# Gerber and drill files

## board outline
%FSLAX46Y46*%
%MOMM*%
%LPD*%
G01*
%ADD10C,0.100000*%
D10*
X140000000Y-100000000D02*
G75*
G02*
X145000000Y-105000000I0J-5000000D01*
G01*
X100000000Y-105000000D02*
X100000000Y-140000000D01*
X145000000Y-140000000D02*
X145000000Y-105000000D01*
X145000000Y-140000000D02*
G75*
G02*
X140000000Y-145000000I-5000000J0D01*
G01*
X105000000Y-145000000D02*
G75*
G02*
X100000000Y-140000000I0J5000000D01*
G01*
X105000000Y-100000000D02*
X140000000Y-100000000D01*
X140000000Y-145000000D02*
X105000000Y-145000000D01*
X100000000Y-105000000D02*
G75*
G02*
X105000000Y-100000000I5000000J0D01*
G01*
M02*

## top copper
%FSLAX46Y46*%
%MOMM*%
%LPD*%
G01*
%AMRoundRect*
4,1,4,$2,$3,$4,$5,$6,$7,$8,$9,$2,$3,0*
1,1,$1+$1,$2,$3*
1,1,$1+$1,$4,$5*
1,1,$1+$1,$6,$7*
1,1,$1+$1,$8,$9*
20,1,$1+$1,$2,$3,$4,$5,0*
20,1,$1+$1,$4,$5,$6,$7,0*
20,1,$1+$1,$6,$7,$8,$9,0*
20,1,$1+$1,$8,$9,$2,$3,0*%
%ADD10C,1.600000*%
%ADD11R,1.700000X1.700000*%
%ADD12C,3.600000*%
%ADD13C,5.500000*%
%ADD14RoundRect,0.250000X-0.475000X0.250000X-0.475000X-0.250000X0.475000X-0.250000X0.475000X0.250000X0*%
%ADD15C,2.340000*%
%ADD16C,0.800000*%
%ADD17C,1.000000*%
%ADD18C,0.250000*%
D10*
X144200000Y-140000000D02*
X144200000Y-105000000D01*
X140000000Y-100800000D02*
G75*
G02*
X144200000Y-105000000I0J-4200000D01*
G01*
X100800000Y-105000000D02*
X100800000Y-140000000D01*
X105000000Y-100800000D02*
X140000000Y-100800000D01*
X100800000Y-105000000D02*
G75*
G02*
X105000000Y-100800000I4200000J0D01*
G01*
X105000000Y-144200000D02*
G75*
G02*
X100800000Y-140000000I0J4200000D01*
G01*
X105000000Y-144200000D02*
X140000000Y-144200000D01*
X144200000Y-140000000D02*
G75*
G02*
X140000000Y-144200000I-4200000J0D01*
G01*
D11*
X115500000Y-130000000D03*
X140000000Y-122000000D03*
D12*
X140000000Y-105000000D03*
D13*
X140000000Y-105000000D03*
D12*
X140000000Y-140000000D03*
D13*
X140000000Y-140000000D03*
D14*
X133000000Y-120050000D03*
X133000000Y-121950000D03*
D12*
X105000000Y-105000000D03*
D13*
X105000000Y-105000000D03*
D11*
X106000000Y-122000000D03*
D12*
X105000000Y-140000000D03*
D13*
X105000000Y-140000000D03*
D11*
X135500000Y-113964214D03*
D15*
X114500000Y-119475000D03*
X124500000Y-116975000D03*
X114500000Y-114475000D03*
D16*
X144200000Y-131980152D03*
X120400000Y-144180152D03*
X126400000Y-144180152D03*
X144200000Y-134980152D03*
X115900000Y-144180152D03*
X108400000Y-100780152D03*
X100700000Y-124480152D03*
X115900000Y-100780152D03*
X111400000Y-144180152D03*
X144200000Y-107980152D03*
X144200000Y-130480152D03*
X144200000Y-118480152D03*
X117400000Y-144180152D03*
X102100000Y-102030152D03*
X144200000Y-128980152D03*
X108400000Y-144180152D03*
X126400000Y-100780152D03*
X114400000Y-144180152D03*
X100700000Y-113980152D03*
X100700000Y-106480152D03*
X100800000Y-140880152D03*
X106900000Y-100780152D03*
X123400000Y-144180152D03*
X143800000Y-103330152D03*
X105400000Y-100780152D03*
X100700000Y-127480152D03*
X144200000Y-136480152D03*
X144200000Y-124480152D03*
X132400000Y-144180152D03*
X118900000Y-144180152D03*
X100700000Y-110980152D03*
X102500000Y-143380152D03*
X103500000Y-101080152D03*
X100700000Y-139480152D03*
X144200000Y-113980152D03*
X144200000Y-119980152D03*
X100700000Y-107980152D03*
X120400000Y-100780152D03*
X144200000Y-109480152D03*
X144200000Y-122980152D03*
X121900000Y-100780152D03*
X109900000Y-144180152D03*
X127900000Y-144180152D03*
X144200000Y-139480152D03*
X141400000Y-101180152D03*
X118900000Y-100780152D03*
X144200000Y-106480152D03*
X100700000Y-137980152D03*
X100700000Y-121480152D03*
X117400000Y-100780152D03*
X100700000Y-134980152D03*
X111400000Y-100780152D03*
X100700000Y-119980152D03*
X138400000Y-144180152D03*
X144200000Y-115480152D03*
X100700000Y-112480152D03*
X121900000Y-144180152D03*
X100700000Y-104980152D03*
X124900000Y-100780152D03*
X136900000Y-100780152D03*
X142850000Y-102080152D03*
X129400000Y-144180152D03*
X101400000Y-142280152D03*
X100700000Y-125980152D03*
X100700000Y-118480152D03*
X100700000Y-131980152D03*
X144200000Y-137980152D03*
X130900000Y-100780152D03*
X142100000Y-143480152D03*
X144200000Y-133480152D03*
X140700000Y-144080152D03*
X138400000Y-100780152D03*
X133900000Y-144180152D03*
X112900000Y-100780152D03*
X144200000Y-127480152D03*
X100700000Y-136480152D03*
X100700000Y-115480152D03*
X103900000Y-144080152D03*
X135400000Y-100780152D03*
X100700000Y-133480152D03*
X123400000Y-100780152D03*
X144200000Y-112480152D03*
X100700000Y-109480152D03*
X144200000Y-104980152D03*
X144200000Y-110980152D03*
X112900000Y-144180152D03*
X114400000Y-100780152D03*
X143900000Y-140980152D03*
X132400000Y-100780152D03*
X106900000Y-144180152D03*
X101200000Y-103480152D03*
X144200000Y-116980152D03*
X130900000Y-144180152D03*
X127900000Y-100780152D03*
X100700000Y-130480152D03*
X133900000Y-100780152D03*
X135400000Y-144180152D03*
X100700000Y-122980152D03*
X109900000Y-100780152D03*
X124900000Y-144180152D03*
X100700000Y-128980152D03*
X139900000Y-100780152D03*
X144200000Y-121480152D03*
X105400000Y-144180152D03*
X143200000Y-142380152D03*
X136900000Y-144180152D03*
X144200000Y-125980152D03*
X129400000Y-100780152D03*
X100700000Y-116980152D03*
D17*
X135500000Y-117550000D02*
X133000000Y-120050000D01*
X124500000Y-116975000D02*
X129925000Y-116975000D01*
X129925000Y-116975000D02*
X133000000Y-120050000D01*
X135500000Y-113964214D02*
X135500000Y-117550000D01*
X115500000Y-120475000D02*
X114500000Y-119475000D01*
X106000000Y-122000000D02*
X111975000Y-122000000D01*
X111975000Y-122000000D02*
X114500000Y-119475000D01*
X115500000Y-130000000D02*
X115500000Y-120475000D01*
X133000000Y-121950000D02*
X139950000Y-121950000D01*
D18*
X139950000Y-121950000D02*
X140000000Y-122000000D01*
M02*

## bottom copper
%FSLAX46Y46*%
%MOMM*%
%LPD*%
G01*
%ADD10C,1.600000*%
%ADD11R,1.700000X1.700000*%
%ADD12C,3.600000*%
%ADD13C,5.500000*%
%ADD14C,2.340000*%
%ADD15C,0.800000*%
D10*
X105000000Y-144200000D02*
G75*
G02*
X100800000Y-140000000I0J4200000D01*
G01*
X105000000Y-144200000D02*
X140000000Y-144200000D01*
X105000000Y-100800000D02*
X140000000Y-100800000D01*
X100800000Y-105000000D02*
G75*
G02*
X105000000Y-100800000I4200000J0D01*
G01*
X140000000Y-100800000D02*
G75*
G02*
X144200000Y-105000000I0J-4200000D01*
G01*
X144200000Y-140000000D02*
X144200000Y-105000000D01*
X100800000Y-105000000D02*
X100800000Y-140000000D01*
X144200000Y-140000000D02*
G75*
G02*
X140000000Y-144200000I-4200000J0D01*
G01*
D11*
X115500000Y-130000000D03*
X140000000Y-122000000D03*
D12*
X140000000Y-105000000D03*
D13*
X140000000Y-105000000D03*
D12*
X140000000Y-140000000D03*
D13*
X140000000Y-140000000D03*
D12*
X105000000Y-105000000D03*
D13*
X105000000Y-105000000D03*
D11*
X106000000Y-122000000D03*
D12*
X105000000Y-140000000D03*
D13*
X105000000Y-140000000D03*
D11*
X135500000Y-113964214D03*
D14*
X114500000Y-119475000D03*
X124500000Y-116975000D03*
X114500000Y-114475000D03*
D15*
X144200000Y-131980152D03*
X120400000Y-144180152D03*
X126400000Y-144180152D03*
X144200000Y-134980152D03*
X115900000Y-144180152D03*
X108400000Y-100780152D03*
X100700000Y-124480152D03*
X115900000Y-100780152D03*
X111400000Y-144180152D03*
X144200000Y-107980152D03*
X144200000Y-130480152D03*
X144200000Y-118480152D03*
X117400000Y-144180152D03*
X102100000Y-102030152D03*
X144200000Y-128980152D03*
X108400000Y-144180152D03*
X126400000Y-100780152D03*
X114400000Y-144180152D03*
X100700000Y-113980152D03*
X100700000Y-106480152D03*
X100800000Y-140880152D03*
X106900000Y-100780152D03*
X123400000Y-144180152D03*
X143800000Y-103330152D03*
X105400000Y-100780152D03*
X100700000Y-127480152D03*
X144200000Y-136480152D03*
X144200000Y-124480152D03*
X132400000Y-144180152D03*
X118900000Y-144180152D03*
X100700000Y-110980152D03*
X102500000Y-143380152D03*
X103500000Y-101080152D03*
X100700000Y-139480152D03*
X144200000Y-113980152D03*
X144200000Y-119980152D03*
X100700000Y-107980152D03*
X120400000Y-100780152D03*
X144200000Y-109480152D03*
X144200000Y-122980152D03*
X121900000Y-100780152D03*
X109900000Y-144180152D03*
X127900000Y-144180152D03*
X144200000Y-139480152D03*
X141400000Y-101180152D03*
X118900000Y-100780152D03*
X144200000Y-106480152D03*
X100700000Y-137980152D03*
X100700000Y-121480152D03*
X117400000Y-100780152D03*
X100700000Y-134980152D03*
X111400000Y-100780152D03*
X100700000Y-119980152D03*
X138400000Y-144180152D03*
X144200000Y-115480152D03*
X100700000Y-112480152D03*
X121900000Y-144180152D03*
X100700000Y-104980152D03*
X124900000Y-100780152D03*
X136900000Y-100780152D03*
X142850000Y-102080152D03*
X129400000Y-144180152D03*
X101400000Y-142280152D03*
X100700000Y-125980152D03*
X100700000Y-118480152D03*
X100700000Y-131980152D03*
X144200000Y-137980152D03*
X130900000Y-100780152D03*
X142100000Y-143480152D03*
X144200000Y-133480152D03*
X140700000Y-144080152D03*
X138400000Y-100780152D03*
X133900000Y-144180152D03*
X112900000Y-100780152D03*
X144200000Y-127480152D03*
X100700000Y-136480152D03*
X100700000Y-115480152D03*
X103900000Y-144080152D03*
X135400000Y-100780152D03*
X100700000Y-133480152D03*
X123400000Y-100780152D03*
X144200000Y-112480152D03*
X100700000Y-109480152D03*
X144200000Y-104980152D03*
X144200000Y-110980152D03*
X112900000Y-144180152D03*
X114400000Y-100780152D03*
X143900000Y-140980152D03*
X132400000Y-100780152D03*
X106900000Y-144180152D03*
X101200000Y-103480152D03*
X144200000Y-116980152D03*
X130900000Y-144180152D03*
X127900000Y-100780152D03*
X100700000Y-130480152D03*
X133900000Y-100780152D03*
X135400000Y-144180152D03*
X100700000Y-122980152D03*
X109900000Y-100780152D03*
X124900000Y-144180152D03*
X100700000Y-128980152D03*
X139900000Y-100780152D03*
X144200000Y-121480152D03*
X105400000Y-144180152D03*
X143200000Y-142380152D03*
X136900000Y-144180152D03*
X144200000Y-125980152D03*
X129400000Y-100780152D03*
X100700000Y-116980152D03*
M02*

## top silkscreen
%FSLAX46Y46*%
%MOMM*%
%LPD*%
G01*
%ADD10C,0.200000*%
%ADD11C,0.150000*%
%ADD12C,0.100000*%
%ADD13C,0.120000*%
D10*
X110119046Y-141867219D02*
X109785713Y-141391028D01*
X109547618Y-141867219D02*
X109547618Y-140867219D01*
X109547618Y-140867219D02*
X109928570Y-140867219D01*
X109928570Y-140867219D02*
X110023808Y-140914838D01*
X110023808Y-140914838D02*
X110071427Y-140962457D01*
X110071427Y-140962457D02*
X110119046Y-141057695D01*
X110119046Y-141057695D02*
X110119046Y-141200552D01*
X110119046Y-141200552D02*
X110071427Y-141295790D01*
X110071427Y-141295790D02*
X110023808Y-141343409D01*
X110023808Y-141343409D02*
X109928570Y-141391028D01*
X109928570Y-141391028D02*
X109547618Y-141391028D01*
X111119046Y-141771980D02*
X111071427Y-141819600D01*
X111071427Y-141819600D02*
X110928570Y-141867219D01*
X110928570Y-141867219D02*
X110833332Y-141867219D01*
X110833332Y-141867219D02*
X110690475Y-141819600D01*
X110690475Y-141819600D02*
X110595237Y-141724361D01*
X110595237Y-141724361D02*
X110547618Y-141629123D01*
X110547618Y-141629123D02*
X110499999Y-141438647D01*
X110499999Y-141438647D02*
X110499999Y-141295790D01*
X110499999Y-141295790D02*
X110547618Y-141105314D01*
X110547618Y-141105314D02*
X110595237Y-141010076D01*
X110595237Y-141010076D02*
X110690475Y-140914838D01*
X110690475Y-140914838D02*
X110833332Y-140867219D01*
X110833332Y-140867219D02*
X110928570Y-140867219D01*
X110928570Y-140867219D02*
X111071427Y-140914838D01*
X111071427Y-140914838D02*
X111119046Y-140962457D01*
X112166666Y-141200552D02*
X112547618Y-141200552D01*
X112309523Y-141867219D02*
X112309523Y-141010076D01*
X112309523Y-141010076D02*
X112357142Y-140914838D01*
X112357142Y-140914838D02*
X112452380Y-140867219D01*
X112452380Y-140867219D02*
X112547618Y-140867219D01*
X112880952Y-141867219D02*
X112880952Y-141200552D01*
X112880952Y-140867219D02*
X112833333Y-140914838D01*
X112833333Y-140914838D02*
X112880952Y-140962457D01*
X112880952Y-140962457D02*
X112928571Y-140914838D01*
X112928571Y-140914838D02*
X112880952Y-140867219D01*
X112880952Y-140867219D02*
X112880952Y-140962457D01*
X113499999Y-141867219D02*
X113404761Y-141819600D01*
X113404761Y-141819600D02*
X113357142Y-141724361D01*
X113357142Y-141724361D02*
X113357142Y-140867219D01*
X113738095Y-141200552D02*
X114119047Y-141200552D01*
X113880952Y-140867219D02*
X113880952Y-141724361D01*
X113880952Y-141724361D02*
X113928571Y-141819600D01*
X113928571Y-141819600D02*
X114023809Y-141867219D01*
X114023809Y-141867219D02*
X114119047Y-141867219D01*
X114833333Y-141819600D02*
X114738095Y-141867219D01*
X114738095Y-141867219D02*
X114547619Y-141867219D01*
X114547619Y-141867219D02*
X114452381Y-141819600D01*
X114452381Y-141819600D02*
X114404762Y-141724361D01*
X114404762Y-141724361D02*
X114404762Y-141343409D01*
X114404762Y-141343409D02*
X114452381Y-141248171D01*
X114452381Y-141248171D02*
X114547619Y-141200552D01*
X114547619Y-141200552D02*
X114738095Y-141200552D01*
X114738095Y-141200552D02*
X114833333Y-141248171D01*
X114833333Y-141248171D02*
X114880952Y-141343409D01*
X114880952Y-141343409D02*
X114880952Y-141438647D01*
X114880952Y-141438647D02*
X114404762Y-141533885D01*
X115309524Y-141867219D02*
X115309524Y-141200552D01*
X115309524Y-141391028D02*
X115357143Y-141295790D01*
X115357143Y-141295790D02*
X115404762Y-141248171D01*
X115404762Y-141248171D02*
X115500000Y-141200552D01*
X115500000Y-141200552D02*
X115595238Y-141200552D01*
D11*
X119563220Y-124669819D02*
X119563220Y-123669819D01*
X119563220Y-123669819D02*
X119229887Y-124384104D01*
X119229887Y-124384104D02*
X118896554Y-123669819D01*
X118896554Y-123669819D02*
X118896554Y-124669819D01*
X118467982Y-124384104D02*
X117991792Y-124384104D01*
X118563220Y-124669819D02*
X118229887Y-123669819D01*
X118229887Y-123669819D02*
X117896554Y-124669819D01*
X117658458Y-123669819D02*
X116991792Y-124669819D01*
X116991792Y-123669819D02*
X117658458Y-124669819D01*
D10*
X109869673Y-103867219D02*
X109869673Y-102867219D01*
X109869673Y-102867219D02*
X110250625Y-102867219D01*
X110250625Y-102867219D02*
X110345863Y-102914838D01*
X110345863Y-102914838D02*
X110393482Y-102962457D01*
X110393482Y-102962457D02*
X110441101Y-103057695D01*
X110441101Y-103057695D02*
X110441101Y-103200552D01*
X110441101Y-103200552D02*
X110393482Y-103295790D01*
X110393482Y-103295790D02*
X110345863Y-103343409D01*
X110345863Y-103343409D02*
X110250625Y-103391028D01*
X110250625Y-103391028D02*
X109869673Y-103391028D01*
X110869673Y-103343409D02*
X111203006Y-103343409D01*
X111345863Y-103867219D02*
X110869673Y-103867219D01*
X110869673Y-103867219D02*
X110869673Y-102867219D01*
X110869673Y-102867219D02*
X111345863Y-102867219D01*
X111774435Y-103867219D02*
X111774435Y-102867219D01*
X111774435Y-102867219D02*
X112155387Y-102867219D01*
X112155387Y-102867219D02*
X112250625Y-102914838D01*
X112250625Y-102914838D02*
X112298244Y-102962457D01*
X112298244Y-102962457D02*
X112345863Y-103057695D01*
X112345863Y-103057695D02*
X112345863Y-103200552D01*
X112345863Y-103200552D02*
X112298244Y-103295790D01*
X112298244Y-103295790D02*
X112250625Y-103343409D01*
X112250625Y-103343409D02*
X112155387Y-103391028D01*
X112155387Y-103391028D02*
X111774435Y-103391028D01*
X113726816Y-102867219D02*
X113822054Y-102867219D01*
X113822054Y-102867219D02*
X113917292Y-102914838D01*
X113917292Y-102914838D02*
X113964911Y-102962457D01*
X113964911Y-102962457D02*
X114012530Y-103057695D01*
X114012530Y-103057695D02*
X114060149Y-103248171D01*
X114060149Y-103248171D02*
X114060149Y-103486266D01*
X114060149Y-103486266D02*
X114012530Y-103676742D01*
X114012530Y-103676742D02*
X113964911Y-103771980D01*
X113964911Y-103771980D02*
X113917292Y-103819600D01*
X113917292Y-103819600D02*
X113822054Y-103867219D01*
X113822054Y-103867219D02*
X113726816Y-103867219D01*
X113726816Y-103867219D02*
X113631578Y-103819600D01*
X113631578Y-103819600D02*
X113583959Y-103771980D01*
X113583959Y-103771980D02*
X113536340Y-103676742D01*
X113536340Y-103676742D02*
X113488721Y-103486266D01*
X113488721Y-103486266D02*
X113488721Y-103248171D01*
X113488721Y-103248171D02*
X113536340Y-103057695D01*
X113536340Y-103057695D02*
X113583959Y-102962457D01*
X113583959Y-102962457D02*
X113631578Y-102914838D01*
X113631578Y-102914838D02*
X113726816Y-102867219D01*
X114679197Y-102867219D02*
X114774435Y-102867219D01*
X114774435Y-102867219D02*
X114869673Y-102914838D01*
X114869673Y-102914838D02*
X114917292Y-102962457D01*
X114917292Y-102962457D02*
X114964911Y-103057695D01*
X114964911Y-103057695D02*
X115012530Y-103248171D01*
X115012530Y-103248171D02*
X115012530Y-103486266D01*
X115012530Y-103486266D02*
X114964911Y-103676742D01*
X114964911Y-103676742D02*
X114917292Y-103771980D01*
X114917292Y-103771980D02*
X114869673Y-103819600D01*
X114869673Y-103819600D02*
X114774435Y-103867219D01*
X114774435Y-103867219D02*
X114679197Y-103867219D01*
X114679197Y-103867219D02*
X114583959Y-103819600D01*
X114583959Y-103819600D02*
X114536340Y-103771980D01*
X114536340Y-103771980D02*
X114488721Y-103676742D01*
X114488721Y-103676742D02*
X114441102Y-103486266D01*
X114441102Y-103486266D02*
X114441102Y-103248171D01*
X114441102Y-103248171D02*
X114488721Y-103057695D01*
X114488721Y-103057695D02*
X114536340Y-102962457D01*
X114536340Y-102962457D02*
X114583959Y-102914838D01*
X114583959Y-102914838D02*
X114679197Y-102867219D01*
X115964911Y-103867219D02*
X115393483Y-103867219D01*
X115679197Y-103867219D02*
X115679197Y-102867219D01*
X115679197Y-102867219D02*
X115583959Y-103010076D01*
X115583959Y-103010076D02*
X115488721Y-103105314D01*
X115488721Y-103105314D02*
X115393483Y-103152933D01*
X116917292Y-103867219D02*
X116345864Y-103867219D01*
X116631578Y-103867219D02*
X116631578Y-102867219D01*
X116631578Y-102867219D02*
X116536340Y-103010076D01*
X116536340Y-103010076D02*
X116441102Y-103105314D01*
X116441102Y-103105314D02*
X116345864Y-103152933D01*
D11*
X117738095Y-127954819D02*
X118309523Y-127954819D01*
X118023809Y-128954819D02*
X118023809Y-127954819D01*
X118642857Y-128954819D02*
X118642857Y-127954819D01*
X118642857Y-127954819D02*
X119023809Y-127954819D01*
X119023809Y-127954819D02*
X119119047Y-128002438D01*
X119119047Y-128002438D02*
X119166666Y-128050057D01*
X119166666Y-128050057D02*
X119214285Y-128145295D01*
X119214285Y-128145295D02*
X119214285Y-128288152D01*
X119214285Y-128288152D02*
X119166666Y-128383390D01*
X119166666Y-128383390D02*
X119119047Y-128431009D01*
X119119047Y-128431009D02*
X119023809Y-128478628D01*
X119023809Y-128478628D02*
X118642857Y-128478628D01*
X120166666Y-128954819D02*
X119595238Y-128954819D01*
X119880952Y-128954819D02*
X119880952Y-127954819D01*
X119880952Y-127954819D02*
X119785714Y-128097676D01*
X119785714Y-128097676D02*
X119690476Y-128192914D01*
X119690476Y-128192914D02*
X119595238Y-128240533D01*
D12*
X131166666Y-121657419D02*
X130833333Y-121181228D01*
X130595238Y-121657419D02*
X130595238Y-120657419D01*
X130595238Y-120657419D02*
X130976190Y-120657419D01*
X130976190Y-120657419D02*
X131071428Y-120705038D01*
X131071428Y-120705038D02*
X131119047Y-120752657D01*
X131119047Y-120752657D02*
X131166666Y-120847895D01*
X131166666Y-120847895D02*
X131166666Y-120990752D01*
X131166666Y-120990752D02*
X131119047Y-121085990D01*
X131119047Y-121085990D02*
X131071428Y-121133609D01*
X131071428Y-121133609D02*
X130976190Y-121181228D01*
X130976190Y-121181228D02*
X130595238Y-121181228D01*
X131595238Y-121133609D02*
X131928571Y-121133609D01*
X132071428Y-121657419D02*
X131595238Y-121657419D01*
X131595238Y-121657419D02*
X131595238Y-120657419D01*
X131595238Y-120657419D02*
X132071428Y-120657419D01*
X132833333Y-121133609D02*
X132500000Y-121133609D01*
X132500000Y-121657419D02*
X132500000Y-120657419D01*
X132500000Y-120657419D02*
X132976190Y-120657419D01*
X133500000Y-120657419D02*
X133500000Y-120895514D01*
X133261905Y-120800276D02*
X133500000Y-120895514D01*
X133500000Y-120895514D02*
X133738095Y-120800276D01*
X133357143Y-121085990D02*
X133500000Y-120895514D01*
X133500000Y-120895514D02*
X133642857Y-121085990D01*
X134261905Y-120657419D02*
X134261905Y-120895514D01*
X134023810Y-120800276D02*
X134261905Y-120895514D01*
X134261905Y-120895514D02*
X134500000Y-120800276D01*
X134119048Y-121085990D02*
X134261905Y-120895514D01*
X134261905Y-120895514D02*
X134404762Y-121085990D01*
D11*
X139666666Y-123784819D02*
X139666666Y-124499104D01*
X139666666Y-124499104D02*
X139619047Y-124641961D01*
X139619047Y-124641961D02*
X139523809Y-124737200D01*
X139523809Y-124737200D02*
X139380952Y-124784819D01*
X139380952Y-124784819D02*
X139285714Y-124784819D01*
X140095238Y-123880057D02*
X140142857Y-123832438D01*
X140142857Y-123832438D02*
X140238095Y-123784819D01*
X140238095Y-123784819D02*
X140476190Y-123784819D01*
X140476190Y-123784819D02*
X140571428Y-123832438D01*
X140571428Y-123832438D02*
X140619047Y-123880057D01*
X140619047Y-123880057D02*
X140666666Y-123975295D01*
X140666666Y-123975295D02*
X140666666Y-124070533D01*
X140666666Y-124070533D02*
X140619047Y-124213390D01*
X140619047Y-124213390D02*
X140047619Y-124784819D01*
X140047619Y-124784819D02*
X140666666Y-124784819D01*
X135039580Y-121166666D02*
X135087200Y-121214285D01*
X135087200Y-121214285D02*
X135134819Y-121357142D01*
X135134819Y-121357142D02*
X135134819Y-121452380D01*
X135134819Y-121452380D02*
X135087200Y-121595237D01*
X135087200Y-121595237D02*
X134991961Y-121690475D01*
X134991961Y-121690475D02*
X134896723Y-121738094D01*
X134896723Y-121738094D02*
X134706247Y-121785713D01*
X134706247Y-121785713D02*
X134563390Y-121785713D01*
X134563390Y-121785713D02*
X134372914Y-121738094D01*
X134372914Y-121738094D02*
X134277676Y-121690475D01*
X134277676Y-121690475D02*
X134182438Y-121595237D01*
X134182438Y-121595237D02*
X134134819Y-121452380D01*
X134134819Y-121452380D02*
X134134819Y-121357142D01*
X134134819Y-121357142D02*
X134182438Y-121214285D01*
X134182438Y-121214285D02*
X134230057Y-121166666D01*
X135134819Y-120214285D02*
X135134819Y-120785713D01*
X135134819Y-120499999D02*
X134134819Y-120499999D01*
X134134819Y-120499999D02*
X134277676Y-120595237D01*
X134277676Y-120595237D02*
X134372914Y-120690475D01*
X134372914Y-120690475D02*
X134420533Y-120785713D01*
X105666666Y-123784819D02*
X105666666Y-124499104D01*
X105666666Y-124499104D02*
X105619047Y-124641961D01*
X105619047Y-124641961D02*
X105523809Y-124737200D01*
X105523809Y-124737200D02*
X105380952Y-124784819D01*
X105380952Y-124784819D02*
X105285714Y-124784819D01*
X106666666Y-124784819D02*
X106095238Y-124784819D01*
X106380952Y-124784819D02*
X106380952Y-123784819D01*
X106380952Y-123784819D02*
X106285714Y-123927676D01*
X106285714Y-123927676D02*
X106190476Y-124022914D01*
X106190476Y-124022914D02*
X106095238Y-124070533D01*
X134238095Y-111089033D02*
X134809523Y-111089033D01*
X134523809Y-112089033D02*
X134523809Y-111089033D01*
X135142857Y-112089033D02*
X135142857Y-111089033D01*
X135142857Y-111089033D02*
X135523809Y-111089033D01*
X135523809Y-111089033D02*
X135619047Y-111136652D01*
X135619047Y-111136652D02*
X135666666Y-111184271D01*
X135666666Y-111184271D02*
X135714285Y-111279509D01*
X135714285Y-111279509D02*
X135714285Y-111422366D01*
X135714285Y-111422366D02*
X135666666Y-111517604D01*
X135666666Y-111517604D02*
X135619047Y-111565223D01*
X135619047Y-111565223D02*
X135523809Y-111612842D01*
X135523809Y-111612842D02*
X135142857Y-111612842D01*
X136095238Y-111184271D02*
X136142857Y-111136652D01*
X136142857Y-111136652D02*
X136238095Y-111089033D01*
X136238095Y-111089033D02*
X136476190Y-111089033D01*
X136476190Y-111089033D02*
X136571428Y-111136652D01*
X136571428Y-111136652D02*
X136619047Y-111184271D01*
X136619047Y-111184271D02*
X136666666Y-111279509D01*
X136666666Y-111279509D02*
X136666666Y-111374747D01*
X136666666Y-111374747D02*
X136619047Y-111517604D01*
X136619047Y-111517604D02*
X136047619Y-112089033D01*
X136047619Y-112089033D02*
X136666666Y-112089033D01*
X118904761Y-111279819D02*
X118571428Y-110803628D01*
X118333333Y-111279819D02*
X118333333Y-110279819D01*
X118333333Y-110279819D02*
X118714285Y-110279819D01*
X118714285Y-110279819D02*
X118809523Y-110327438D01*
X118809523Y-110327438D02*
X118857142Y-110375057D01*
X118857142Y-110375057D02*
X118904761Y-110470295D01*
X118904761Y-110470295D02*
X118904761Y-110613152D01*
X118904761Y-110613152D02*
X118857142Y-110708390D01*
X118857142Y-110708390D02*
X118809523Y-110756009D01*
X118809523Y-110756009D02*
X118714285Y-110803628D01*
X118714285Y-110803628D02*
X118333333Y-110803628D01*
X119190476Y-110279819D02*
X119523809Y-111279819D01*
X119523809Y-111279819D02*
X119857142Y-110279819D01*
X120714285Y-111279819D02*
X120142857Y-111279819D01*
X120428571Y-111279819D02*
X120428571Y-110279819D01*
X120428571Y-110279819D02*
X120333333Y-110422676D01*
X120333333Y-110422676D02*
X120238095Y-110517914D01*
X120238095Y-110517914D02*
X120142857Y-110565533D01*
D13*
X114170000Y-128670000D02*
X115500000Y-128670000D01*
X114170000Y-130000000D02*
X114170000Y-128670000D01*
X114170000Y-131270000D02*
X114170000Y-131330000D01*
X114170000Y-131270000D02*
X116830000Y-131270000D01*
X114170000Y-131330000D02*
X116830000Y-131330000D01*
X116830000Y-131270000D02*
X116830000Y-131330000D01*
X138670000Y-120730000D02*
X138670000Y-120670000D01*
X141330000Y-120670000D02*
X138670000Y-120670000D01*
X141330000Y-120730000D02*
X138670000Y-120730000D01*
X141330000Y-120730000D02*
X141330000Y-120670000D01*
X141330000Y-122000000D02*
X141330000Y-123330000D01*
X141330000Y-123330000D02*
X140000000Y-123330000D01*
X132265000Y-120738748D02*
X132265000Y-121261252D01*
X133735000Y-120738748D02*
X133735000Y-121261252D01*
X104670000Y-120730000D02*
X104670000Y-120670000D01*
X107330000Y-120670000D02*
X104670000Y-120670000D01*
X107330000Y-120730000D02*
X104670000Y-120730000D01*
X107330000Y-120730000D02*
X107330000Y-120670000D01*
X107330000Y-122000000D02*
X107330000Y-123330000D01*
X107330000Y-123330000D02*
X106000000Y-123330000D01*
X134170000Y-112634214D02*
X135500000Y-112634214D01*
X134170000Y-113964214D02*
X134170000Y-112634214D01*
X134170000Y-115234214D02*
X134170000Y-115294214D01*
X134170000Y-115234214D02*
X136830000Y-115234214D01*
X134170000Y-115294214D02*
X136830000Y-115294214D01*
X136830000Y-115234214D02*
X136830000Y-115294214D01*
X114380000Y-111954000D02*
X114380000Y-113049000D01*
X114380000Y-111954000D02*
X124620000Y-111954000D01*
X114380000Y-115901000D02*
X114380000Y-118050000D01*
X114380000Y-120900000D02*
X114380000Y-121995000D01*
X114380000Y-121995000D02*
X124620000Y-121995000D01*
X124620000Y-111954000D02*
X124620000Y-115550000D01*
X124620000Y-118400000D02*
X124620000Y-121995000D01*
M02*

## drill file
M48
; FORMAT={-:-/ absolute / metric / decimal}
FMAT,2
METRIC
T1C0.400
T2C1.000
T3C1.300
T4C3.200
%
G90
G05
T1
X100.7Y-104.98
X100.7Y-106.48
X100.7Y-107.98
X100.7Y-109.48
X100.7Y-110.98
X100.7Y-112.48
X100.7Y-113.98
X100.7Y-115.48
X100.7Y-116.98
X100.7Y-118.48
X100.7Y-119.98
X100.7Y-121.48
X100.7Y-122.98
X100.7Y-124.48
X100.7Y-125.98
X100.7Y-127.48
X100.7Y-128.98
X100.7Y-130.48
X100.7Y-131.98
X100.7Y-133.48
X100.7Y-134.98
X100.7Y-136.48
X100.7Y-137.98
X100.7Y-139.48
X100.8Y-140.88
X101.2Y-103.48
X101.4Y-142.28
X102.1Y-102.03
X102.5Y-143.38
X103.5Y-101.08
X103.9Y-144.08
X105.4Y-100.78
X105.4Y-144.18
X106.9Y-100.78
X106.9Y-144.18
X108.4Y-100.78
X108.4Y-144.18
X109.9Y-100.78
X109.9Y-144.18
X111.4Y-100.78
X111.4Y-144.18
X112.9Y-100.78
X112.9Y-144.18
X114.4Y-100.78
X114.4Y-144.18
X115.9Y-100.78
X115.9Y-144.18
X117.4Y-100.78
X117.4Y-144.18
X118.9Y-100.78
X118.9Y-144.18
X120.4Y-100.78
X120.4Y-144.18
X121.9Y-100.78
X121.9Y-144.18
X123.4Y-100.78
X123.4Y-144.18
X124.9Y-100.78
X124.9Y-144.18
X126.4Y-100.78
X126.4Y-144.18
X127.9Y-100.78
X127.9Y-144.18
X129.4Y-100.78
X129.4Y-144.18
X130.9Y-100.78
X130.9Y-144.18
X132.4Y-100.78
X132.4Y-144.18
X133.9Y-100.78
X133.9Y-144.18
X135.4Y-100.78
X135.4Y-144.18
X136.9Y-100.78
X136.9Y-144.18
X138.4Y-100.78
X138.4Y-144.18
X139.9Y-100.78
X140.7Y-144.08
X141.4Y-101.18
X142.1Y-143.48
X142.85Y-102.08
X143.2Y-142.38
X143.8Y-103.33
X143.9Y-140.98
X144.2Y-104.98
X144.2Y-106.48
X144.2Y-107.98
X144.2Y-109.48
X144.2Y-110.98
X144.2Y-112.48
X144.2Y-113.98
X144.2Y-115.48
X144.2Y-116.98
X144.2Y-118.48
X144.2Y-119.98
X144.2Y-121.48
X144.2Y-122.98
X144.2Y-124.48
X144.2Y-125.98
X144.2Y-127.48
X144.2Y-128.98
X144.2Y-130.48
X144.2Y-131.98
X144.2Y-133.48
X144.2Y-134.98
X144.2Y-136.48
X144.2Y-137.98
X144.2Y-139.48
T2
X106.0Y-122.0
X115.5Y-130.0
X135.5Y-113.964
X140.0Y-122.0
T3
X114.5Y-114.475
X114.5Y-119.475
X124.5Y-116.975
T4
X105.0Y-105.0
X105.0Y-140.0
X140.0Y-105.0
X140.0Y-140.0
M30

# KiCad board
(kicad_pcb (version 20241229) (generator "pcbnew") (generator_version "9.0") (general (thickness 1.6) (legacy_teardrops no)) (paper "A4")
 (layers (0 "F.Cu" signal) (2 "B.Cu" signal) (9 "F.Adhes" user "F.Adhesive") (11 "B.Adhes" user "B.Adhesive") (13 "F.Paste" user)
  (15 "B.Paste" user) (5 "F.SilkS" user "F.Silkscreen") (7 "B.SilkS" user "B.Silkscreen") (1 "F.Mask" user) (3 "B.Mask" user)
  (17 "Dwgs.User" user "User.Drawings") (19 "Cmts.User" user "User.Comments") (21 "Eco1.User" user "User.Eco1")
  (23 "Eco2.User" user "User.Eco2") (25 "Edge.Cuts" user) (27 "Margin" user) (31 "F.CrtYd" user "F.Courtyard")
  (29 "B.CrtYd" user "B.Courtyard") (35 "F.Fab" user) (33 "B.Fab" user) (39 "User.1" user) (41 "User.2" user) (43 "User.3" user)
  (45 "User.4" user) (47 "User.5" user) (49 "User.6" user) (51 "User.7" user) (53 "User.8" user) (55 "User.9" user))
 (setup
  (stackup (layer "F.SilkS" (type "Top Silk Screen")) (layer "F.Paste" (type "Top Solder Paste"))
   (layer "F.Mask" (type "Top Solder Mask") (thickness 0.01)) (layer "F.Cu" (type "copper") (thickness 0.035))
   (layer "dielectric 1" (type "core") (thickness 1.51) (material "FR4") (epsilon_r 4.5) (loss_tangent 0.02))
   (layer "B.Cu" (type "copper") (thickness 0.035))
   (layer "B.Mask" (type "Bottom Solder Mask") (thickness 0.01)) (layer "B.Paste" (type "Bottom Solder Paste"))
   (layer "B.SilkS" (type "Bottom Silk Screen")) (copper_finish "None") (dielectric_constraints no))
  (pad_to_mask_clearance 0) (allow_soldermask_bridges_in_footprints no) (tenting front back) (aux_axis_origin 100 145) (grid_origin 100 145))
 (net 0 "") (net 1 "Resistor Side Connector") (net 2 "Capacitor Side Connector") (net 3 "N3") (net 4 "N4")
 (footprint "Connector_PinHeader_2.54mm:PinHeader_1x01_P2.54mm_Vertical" (layer "F.Cu") (at 115.5 130)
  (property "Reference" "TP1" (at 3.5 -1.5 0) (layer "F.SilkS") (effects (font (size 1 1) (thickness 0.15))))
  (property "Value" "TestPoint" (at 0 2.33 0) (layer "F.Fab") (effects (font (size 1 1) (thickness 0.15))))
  (fp_line (start -1.33 -1.33) (end 0 -1.33) (stroke (width 0.12) (type solid)) (layer "F.SilkS"))
  (fp_line (start -1.33 0) (end -1.33 -1.33) (stroke (width 0.12) (type solid)) (layer "F.SilkS"))
  (fp_line (start -1.33 1.27) (end -1.33 1.33) (stroke (width 0.12) (type solid)) (layer "F.SilkS"))
  (fp_line (start -1.33 1.27) (end 1.33 1.27) (stroke (width 0.12) (type solid)) (layer "F.SilkS"))
  (fp_line (start -1.33 1.33) (end 1.33 1.33) (stroke (width 0.12) (type solid)) (layer "F.SilkS"))
  (fp_line (start 1.33 1.27) (end 1.33 1.33) (stroke (width 0.12) (type solid)) (layer "F.SilkS"))
  (pad "1" thru_hole rect (at 0 0) (size 1.7 1.7) (drill 1) (layers "*.Cu" "*.Mask") (remove_unused_layers no)
   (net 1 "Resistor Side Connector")))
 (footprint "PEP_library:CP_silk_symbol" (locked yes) (layer "F.Cu") (at 129.5 118.7 90)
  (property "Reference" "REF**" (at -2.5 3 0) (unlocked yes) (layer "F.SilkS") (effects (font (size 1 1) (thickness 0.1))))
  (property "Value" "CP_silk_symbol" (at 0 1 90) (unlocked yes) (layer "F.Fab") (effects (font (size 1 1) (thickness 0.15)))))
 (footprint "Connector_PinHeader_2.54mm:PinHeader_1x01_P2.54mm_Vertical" (layer "F.Cu") (at 140 122 180)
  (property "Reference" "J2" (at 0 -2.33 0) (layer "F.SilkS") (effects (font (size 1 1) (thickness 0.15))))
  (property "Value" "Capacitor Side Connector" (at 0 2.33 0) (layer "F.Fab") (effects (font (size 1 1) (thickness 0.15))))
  (fp_line (start 1.33 1.27) (end 1.33 1.33) (stroke (width 0.12) (type solid)) (layer "F.SilkS"))
  (fp_line (start -1.33 1.33) (end 1.33 1.33) (stroke (width 0.12) (type solid)) (layer "F.SilkS"))
  (fp_line (start -1.33 1.27) (end 1.33 1.27) (stroke (width 0.12) (type solid)) (layer "F.SilkS"))
  (fp_line (start -1.33 1.27) (end -1.33 1.33) (stroke (width 0.12) (type solid)) (layer "F.SilkS"))
  (fp_line (start -1.33 0) (end -1.33 -1.33) (stroke (width 0.12) (type solid)) (layer "F.SilkS"))
  (fp_line (start -1.33 -1.33) (end 0 -1.33) (stroke (width 0.12) (type solid)) (layer "F.SilkS"))
  (pad "1" thru_hole rect (at 0 0 180) (size 1.7 1.7) (drill 1) (layers "*.Cu" "*.Mask") (remove_unused_layers no)
   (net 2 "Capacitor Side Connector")))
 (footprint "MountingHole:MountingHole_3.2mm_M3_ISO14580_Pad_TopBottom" (layer "F.Cu") (at 140 105)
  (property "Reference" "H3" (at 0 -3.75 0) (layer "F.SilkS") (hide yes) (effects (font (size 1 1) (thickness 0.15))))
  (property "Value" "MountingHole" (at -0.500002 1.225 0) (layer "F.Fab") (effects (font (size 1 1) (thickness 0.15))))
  (pad "1" thru_hole circle (at 0 0) (size 3.6 3.6) (drill 3.2) (layers "*.Cu" "*.Mask") (remove_unused_layers no))
  (pad "1" connect circle (at 0 0) (size 5.5 5.5) (layers "F.Cu" "F.Mask"))
  (pad "1" connect circle (at 0 0) (size 5.5 5.5) (layers "B.Cu" "B.Mask")))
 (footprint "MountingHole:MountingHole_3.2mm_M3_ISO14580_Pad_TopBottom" (layer "F.Cu") (at 140 140)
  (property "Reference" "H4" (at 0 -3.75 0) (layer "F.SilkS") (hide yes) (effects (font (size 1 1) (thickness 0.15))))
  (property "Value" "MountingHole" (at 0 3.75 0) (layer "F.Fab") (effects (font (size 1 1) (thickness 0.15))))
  (pad "1" thru_hole circle (at 0 0) (size 3.6 3.6) (drill 3.2) (layers "*.Cu" "*.Mask") (remove_unused_layers no))
  (pad "1" connect circle (at 0 0) (size 5.5 5.5) (layers "F.Cu" "F.Mask"))
  (pad "1" connect circle (at 0 0) (size 5.5 5.5) (layers "B.Cu" "B.Mask")))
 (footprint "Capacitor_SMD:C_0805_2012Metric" (layer "F.Cu") (at 133 121 -90)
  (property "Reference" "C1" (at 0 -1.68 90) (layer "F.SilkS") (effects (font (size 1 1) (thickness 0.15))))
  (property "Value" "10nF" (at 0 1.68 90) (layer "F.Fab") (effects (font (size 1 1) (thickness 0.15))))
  (fp_line (start -0.261252 0.735) (end 0.261252 0.735) (stroke (width 0.12) (type solid)) (layer "F.SilkS"))
  (fp_line (start -0.261252 -0.735) (end 0.261252 -0.735) (stroke (width 0.12) (type solid)) (layer "F.SilkS"))
  (pad "1" smd roundrect (at -0.95 0 270) (size 1 1.45) (layers "F.Cu" "F.Mask" "F.Paste") (roundrect_rratio 0.25) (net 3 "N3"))
  (pad "2" smd roundrect (at 0.95 0 270) (size 1 1.45) (layers "F.Cu" "F.Mask" "F.Paste") (roundrect_rratio 0.25)
   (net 2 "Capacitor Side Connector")))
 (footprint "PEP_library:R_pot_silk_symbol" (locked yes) (layer "F.Cu") (at 124.2125 109.4375 -90)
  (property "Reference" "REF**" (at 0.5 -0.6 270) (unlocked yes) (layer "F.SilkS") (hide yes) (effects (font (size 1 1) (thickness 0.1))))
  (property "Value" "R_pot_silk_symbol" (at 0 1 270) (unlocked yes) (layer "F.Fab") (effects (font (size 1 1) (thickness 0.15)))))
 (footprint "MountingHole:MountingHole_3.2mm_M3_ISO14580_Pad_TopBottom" (layer "F.Cu") (at 105 105)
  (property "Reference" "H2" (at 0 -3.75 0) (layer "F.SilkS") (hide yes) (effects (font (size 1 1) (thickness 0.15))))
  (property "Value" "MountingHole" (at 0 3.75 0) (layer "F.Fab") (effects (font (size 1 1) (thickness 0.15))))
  (pad "1" thru_hole circle (at 0 0) (size 3.6 3.6) (drill 3.2) (layers "*.Cu" "*.Mask") (remove_unused_layers no))
  (pad "1" connect circle (at 0 0) (size 5.5 5.5) (layers "F.Cu" "F.Mask"))
  (pad "1" connect circle (at 0 0) (size 5.5 5.5) (layers "B.Cu" "B.Mask")))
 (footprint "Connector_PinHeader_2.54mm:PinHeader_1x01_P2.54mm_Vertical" (layer "F.Cu") (at 106 122 180)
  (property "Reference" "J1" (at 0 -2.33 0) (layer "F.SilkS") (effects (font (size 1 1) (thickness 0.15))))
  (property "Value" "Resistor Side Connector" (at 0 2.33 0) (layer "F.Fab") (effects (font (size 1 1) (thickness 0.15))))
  (fp_line (start 1.33 1.27) (end 1.33 1.33) (stroke (width 0.12) (type solid)) (layer "F.SilkS"))
  (fp_line (start -1.33 1.33) (end 1.33 1.33) (stroke (width 0.12) (type solid)) (layer "F.SilkS"))
  (fp_line (start -1.33 1.27) (end 1.33 1.27) (stroke (width 0.12) (type solid)) (layer "F.SilkS"))
  (fp_line (start -1.33 1.27) (end -1.33 1.33) (stroke (width 0.12) (type solid)) (layer "F.SilkS"))
  (fp_line (start -1.33 0) (end -1.33 -1.33) (stroke (width 0.12) (type solid)) (layer "F.SilkS"))
  (fp_line (start -1.33 -1.33) (end 0 -1.33) (stroke (width 0.12) (type solid)) (layer "F.SilkS"))
  (pad "1" thru_hole rect (at 0 0 180) (size 1.7 1.7) (drill 1) (layers "*.Cu" "*.Mask") (remove_unused_layers no)
   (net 1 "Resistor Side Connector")))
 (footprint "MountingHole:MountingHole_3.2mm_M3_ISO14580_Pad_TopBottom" (layer "F.Cu") (at 105 140 -90)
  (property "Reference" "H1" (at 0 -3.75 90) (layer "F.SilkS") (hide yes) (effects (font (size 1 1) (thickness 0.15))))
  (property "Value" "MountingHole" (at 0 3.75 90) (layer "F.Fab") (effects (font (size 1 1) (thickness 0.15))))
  (pad "1" thru_hole circle (at 0 0 270) (size 3.6 3.6) (drill 3.2) (layers "*.Cu" "*.Mask") (remove_unused_layers no))
  (pad "1" connect circle (at 0 0 270) (size 5.5 5.5) (layers "F.Cu" "F.Mask"))
  (pad "1" connect circle (at 0 0 270) (size 5.5 5.5) (layers "B.Cu" "B.Mask")))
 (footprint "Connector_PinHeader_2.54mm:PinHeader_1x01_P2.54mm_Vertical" (layer "F.Cu") (at 135.5 113.964214)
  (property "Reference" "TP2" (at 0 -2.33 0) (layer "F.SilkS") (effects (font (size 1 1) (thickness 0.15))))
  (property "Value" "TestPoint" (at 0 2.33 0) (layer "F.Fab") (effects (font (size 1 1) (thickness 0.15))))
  (fp_line (start -1.33 -1.33) (end 0 -1.33) (stroke (width 0.12) (type solid)) (layer "F.SilkS"))
  (fp_line (start -1.33 0) (end -1.33 -1.33) (stroke (width 0.12) (type solid)) (layer "F.SilkS"))
  (fp_line (start -1.33 1.27) (end -1.33 1.33) (stroke (width 0.12) (type solid)) (layer "F.SilkS"))
  (fp_line (start -1.33 1.27) (end 1.33 1.27) (stroke (width 0.12) (type solid)) (layer "F.SilkS"))
  (fp_line (start -1.33 1.33) (end 1.33 1.33) (stroke (width 0.12) (type solid)) (layer "F.SilkS"))
  (fp_line (start 1.33 1.27) (end 1.33 1.33) (stroke (width 0.12) (type solid)) (layer "F.SilkS"))
  (pad "1" thru_hole rect (at 0 0) (size 1.7 1.7) (drill 1) (layers "*.Cu" "*.Mask") (remove_unused_layers no) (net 3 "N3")))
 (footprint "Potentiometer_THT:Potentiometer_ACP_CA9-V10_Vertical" (layer "F.Cu") (at 114.5 119.475)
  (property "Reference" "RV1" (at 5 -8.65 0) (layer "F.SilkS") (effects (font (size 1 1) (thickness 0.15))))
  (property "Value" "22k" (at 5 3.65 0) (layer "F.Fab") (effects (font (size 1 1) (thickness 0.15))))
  (fp_line (start -0.12 -7.521) (end -0.12 -6.426) (stroke (width 0.12) (type solid)) (layer "F.SilkS"))
  (fp_line (start -0.12 -7.521) (end 10.12 -7.521) (stroke (width 0.12) (type solid)) (layer "F.SilkS"))
  (fp_line (start -0.12 -3.574) (end -0.12 -1.425) (stroke (width 0.12) (type solid)) (layer "F.SilkS"))
  (fp_line (start -0.12 1.425) (end -0.12 2.52) (stroke (width 0.12) (type solid)) (layer "F.SilkS"))
  (fp_line (start -0.12 2.52) (end 10.12 2.52) (stroke (width 0.12) (type solid)) (layer "F.SilkS"))
  (fp_line (start 10.12 -7.521) (end 10.12 -3.925) (stroke (width 0.12) (type solid)) (layer "F.SilkS"))
  (fp_line (start 10.12 -1.075) (end 10.12 2.52) (stroke (width 0.12) (type solid)) (layer "F.SilkS"))
  (pad "1" thru_hole circle (at 0 0) (size 2.34 2.34) (drill 1.3) (layers "*.Cu" "*.Mask") (remove_unused_layers no)
   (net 1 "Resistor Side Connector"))
  (pad "2" thru_hole circle (at 10 -2.5) (size 2.34 2.34) (drill 1.3) (layers "*.Cu" "*.Mask") (remove_unused_layers no) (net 3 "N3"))
  (pad "3" thru_hole circle (at 0 -5) (size 2.34 2.34) (drill 1.3) (layers "*.Cu" "*.Mask") (remove_unused_layers no) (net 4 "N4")))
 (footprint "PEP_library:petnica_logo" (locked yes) (layer "B.Cu") (at 127.5 132.5 180)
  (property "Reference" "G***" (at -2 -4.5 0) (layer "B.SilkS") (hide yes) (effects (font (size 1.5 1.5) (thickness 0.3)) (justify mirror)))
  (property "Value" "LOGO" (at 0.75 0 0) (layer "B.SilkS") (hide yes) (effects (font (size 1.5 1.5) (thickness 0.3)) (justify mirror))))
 (gr_line (start 144.2 140) (end 144.2 105) (stroke (width 1.6) (type solid)) (locked yes) (layer "F.Cu") (net 4))
 (gr_arc (start 140 100.8) (mid 142.969848 102.030152) (end 144.2 105) (stroke (width 1.6) (type default)) (locked yes) (layer "F.Cu")
  (net 4))
 (gr_line (start 100.8 105) (end 100.8 140) (stroke (width 1.6) (type solid)) (locked yes) (layer "F.Cu") (net 4))
 (gr_line (start 105 100.8) (end 140 100.8) (stroke (width 1.6) (type solid)) (locked yes) (layer "F.Cu") (net 4))
 (gr_arc (start 100.8 105) (mid 102.030152 102.030152) (end 105 100.8) (stroke (width 1.6) (type solid)) (locked yes) (layer "F.Cu") (net 4))
 (gr_arc (start 105 144.2) (mid 102.030152 142.969848) (end 100.8 140) (stroke (width 1.6) (type solid)) (locked yes) (layer "F.Cu") (net 4))
 (gr_line (start 105 144.2) (end 140 144.2) (stroke (width 1.6) (type solid)) (locked yes) (layer "F.Cu") (net 4))
 (gr_arc (start 144.2 140) (mid 142.969848 142.969848) (end 140 144.2) (stroke (width 1.6) (type solid)) (locked yes) (layer "F.Cu") (net 4))
 (gr_arc (start 105 144.2) (mid 102.030154 142.969848) (end 100.8 140) (stroke (width 1.6) (type default)) (locked yes) (layer "B.Cu")
  (net 4))
 (gr_line (start 105 144.2) (end 140 144.2) (stroke (width 1.6) (type default)) (locked yes) (layer "B.Cu") (net 4))
 (gr_line (start 105 100.8) (end 140 100.8) (stroke (width 1.6) (type default)) (locked yes) (layer "B.Cu") (net 4))
 (gr_arc (start 100.8 105) (mid 102.030152 102.030152) (end 105 100.8) (stroke (width 1.6) (type default)) (locked yes) (layer "B.Cu")
  (net 4))
 (gr_arc (start 140 100.8) (mid 142.96985 102.030151) (end 144.2 105) (stroke (width 1.6) (type default)) (locked yes) (layer "B.Cu")
  (net 4))
 (gr_line (start 144.2 140) (end 144.2 105) (stroke (width 1.6) (type default)) (locked yes) (layer "B.Cu") (net 4))
 (gr_line (start 100.8 105) (end 100.8 140) (stroke (width 1.6) (type default)) (locked yes) (layer "B.Cu") (net 4))
 (gr_arc (start 144.2 140) (mid 142.969849 142.969849) (end 140 144.2) (stroke (width 1.6) (type default)) (locked yes) (layer "B.Cu")
  (net 4))
 (gr_arc (start 140 100) (mid 143.535534 101.464466) (end 145 105) (stroke (width 0.1) (type default)) (locked yes) (layer "Edge.Cuts"))
 (gr_line (start 100 105) (end 100 140) (stroke (width 0.1) (type default)) (locked yes) (layer "Edge.Cuts"))
 (gr_line (start 145 140) (end 145 105) (stroke (width 0.1) (type default)) (locked yes) (layer "Edge.Cuts"))
 (gr_arc (start 145 140) (mid 143.535534 143.535534) (end 140 145) (stroke (width 0.1) (type default)) (locked yes) (layer "Edge.Cuts"))
 (gr_arc (start 105 145) (mid 101.464466 143.535534) (end 100 140) (stroke (width 0.1) (type default)) (locked yes) (layer "Edge.Cuts"))
 (gr_line (start 105 100) (end 140 100) (stroke (width 0.1) (type default)) (locked yes) (layer "Edge.Cuts"))
 (gr_line (start 140 145) (end 105 145) (stroke (width 0.1) (type default)) (locked yes) (layer "Edge.Cuts"))
 (gr_arc (start 100 105) (mid 101.464466 101.464466) (end 105 100) (stroke (width 0.1) (type default)) (locked yes) (layer "Edge.Cuts"))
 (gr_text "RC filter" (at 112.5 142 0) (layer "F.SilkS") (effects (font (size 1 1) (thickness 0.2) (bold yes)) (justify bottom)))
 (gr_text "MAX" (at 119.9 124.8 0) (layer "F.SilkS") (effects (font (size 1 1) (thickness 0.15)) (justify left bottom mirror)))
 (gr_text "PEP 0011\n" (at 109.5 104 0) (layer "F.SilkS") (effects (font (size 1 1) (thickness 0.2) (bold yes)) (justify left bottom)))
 (via (at 144.2 131.980152) (size 0.8) (drill 0.4) (layers "F.Cu" "B.Cu") (locked yes) (free yes) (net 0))
 (via (at 120.4 144.180152) (size 0.8) (drill 0.4) (layers "F.Cu" "B.Cu") (locked yes) (free yes) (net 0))
 (via (at 126.4 144.180152) (size 0.8) (drill 0.4) (layers "F.Cu" "B.Cu") (locked yes) (free yes) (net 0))
 (via (at 144.2 134.980152) (size 0.8) (drill 0.4) (layers "F.Cu" "B.Cu") (locked yes) (free yes) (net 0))
 (via (at 115.9 144.180152) (size 0.8) (drill 0.4) (layers "F.Cu" "B.Cu") (locked yes) (free yes) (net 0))
 (via (at 108.4 100.780152) (size 0.8) (drill 0.4) (layers "F.Cu" "B.Cu") (locked yes) (free yes) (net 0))
 (via (at 100.7 124.480152) (size 0.8) (drill 0.4) (layers "F.Cu" "B.Cu") (locked yes) (free yes) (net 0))
 (via (at 115.9 100.780152) (size 0.8) (drill 0.4) (layers "F.Cu" "B.Cu") (locked yes) (free yes) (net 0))
 (via (at 111.4 144.180152) (size 0.8) (drill 0.4) (layers "F.Cu" "B.Cu") (locked yes) (free yes) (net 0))
 (via (at 144.2 107.980152) (size 0.8) (drill 0.4) (layers "F.Cu" "B.Cu") (locked yes) (free yes) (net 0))
 (via (at 144.2 130.480152) (size 0.8) (drill 0.4) (layers "F.Cu" "B.Cu") (locked yes) (free yes) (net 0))
 (via (at 144.2 118.480152) (size 0.8) (drill 0.4) (layers "F.Cu" "B.Cu") (locked yes) (free yes) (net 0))
 (via (at 117.4 144.180152) (size 0.8) (drill 0.4) (layers "F.Cu" "B.Cu") (locked yes) (free yes) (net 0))
 (via (at 102.1 102.030152) (size 0.8) (drill 0.4) (layers "F.Cu" "B.Cu") (locked yes) (free yes) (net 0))
 (via (at 144.2 128.980152) (size 0.8) (drill 0.4) (layers "F.Cu" "B.Cu") (locked yes) (free yes) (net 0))
 (via (at 108.4 144.180152) (size 0.8) (drill 0.4) (layers "F.Cu" "B.Cu") (locked yes) (free yes) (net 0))
 (via (at 126.4 100.780152) (size 0.8) (drill 0.4) (layers "F.Cu" "B.Cu") (locked yes) (free yes) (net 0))
 (via (at 114.4 144.180152) (size 0.8) (drill 0.4) (layers "F.Cu" "B.Cu") (locked yes) (free yes) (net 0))
 (via (at 100.7 113.980152) (size 0.8) (drill 0.4) (layers "F.Cu" "B.Cu") (locked yes) (free yes) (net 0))
 (via (at 100.7 106.480152) (size 0.8) (drill 0.4) (layers "F.Cu" "B.Cu") (locked yes) (free yes) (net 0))
 (via (at 100.8 140.880152) (size 0.8) (drill 0.4) (layers "F.Cu" "B.Cu") (locked yes) (free yes) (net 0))
 (via (at 106.9 100.780152) (size 0.8) (drill 0.4) (layers "F.Cu" "B.Cu") (locked yes) (free yes) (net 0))
 (via (at 123.4 144.180152) (size 0.8) (drill 0.4) (layers "F.Cu" "B.Cu") (locked yes) (free yes) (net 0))
 (via (at 143.8 103.330152) (size 0.8) (drill 0.4) (layers "F.Cu" "B.Cu") (locked yes) (free yes) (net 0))
 (via (at 105.4 100.780152) (size 0.8) (drill 0.4) (layers "F.Cu" "B.Cu") (locked yes) (free yes) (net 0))
 (via (at 100.7 127.480152) (size 0.8) (drill 0.4) (layers "F.Cu" "B.Cu") (locked yes) (free yes) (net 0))
 (via (at 144.2 136.480152) (size 0.8) (drill 0.4) (layers "F.Cu" "B.Cu") (locked yes) (free yes) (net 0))
 (via (at 144.2 124.480152) (size 0.8) (drill 0.4) (layers "F.Cu" "B.Cu") (locked yes) (free yes) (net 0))
 (via (at 132.4 144.180152) (size 0.8) (drill 0.4) (layers "F.Cu" "B.Cu") (locked yes) (free yes) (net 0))
 (via (at 118.9 144.180152) (size 0.8) (drill 0.4) (layers "F.Cu" "B.Cu") (locked yes) (free yes) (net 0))
 (via (at 100.7 110.980152) (size 0.8) (drill 0.4) (layers "F.Cu" "B.Cu") (locked yes) (free yes) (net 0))
 (via (at 102.5 143.380152) (size 0.8) (drill 0.4) (layers "F.Cu" "B.Cu") (locked yes) (free yes) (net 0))
 (via (at 103.5 101.080152) (size 0.8) (drill 0.4) (layers "F.Cu" "B.Cu") (locked yes) (free yes) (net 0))
 (via (at 100.7 139.480152) (size 0.8) (drill 0.4) (layers "F.Cu" "B.Cu") (locked yes) (free yes) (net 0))
 (via (at 144.2 113.980152) (size 0.8) (drill 0.4) (layers "F.Cu" "B.Cu") (locked yes) (free yes) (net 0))
 (via (at 144.2 119.980152) (size 0.8) (drill 0.4) (layers "F.Cu" "B.Cu") (locked yes) (free yes) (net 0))
 (via (at 100.7 107.980152) (size 0.8) (drill 0.4) (layers "F.Cu" "B.Cu") (locked yes) (free yes) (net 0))
 (via (at 120.4 100.780152) (size 0.8) (drill 0.4) (layers "F.Cu" "B.Cu") (locked yes) (free yes) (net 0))
 (via (at 144.2 109.480152) (size 0.8) (drill 0.4) (layers "F.Cu" "B.Cu") (locked yes) (free yes) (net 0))
 (via (at 144.2 122.980152) (size 0.8) (drill 0.4) (layers "F.Cu" "B.Cu") (locked yes) (free yes) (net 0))
 (via (at 121.9 100.780152) (size 0.8) (drill 0.4) (layers "F.Cu" "B.Cu") (locked yes) (free yes) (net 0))
 (via (at 109.9 144.180152) (size 0.8) (drill 0.4) (layers "F.Cu" "B.Cu") (locked yes) (free yes) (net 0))
 (via (at 127.9 144.180152) (size 0.8) (drill 0.4) (layers "F.Cu" "B.Cu") (locked yes) (free yes) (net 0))
 (via (at 144.2 139.480152) (size 0.8) (drill 0.4) (layers "F.Cu" "B.Cu") (locked yes) (free yes) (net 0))
 (via (at 141.4 101.180152) (size 0.8) (drill 0.4) (layers "F.Cu" "B.Cu") (locked yes) (free yes) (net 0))
 (via (at 118.9 100.780152) (size 0.8) (drill 0.4) (layers "F.Cu" "B.Cu") (locked yes) (free yes) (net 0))
 (via (at 144.2 106.480152) (size 0.8) (drill 0.4) (layers "F.Cu" "B.Cu") (locked yes) (free yes) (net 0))
 (via (at 100.7 137.980152) (size 0.8) (drill 0.4) (layers "F.Cu" "B.Cu") (locked yes) (free yes) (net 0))
 (via (at 100.7 121.480152) (size 0.8) (drill 0.4) (layers "F.Cu" "B.Cu") (locked yes) (free yes) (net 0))
 (via (at 117.4 100.780152) (size 0.8) (drill 0.4) (layers "F.Cu" "B.Cu") (locked yes) (free yes) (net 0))
 (via (at 100.7 134.980152) (size 0.8) (drill 0.4) (layers "F.Cu" "B.Cu") (locked yes) (free yes) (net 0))
 (via (at 111.4 100.780152) (size 0.8) (drill 0.4) (layers "F.Cu" "B.Cu") (locked yes) (free yes) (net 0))
 (via (at 100.7 119.980152) (size 0.8) (drill 0.4) (layers "F.Cu" "B.Cu") (locked yes) (free yes) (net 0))
 (via (at 138.4 144.180152) (size 0.8) (drill 0.4) (layers "F.Cu" "B.Cu") (locked yes) (free yes) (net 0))
 (via (at 144.2 115.480152) (size 0.8) (drill 0.4) (layers "F.Cu" "B.Cu") (locked yes) (free yes) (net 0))
 (via (at 100.7 112.480152) (size 0.8) (drill 0.4) (layers "F.Cu" "B.Cu") (locked yes) (free yes) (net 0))
 (via (at 121.9 144.180152) (size 0.8) (drill 0.4) (layers "F.Cu" "B.Cu") (locked yes) (free yes) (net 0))
 (via (at 100.7 104.980152) (size 0.8) (drill 0.4) (layers "F.Cu" "B.Cu") (locked yes) (free yes) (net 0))
 (via (at 124.9 100.780152) (size 0.8) (drill 0.4) (layers "F.Cu" "B.Cu") (locked yes) (free yes) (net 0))
 (via (at 136.9 100.780152) (size 0.8) (drill 0.4) (layers "F.Cu" "B.Cu") (locked yes) (free yes) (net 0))
 (via (at 142.85 102.080152) (size 0.8) (drill 0.4) (layers "F.Cu" "B.Cu") (locked yes) (free yes) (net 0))
 (via (at 129.4 144.180152) (size 0.8) (drill 0.4) (layers "F.Cu" "B.Cu") (locked yes) (free yes) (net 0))
 (via (at 101.4 142.280152) (size 0.8) (drill 0.4) (layers "F.Cu" "B.Cu") (locked yes) (free yes) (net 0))
 (via (at 100.7 125.980152) (size 0.8) (drill 0.4) (layers "F.Cu" "B.Cu") (locked yes) (free yes) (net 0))
 (via (at 100.7 118.480152) (size 0.8) (drill 0.4) (layers "F.Cu" "B.Cu") (locked yes) (free yes) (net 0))
 (via (at 100.7 131.980152) (size 0.8) (drill 0.4) (layers "F.Cu" "B.Cu") (locked yes) (free yes) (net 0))
 (via (at 144.2 137.980152) (size 0.8) (drill 0.4) (layers "F.Cu" "B.Cu") (locked yes) (free yes) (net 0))
 (via (at 130.9 100.780152) (size 0.8) (drill 0.4) (layers "F.Cu" "B.Cu") (locked yes) (free yes) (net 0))
 (via (at 142.1 143.480152) (size 0.8) (drill 0.4) (layers "F.Cu" "B.Cu") (locked yes) (free yes) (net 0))
 (via (at 144.2 133.480152) (size 0.8) (drill 0.4) (layers "F.Cu" "B.Cu") (locked yes) (free yes) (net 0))
 (via (at 140.7 144.080152) (size 0.8) (drill 0.4) (layers "F.Cu" "B.Cu") (locked yes) (free yes) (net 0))
 (via (at 138.4 100.780152) (size 0.8) (drill 0.4) (layers "F.Cu" "B.Cu") (locked yes) (free yes) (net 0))
 (via (at 133.9 144.180152) (size 0.8) (drill 0.4) (layers "F.Cu" "B.Cu") (locked yes) (free yes) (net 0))
 (via (at 112.9 100.780152) (size 0.8) (drill 0.4) (layers "F.Cu" "B.Cu") (locked yes) (free yes) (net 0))
 (via (at 144.2 127.480152) (size 0.8) (drill 0.4) (layers "F.Cu" "B.Cu") (locked yes) (free yes) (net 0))
 (via (at 100.7 136.480152) (size 0.8) (drill 0.4) (layers "F.Cu" "B.Cu") (locked yes) (free yes) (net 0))
 (via (at 100.7 115.480152) (size 0.8) (drill 0.4) (layers "F.Cu" "B.Cu") (locked yes) (free yes) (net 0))
 (via (at 103.9 144.080152) (size 0.8) (drill 0.4) (layers "F.Cu" "B.Cu") (locked yes) (free yes) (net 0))
 (via (at 135.4 100.780152) (size 0.8) (drill 0.4) (layers "F.Cu" "B.Cu") (locked yes) (free yes) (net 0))
 (via (at 100.7 133.480152) (size 0.8) (drill 0.4) (layers "F.Cu" "B.Cu") (locked yes) (free yes) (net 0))
 (via (at 123.4 100.780152) (size 0.8) (drill 0.4) (layers "F.Cu" "B.Cu") (locked yes) (free yes) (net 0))
 (via (at 144.2 112.480152) (size 0.8) (drill 0.4) (layers "F.Cu" "B.Cu") (locked yes) (free yes) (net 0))
 (via (at 100.7 109.480152) (size 0.8) (drill 0.4) (layers "F.Cu" "B.Cu") (locked yes) (free yes) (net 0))
 (via (at 144.2 104.980152) (size 0.8) (drill 0.4) (layers "F.Cu" "B.Cu") (locked yes) (free yes) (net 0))
 (via (at 144.2 110.980152) (size 0.8) (drill 0.4) (layers "F.Cu" "B.Cu") (locked yes) (free yes) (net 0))
 (via (at 112.9 144.180152) (size 0.8) (drill 0.4) (layers "F.Cu" "B.Cu") (locked yes) (free yes) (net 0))
 (via (at 114.4 100.780152) (size 0.8) (drill 0.4) (layers "F.Cu" "B.Cu") (locked yes) (free yes) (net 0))
 (via (at 143.9 140.980152) (size 0.8) (drill 0.4) (layers "F.Cu" "B.Cu") (locked yes) (free yes) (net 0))
 (via (at 132.4 100.780152) (size 0.8) (drill 0.4) (layers "F.Cu" "B.Cu") (locked yes) (free yes) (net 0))
 (via (at 106.9 144.180152) (size 0.8) (drill 0.4) (layers "F.Cu" "B.Cu") (locked yes) (free yes) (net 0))
 (via (at 101.2 103.480152) (size 0.8) (drill 0.4) (layers "F.Cu" "B.Cu") (locked yes) (free yes) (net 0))
 (via (at 144.2 116.980152) (size 0.8) (drill 0.4) (layers "F.Cu" "B.Cu") (locked yes) (free yes) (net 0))
 (via (at 130.9 144.180152) (size 0.8) (drill 0.4) (layers "F.Cu" "B.Cu") (locked yes) (free yes) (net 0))
 (via (at 127.9 100.780152) (size 0.8) (drill 0.4) (layers "F.Cu" "B.Cu") (locked yes) (free yes) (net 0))
 (via (at 100.7 130.480152) (size 0.8) (drill 0.4) (layers "F.Cu" "B.Cu") (locked yes) (free yes) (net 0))
 (via (at 133.9 100.780152) (size 0.8) (drill 0.4) (layers "F.Cu" "B.Cu") (locked yes) (free yes) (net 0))
 (via (at 135.4 144.180152) (size 0.8) (drill 0.4) (layers "F.Cu" "B.Cu") (locked yes) (free yes) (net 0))
 (via (at 100.7 122.980152) (size 0.8) (drill 0.4) (layers "F.Cu" "B.Cu") (locked yes) (free yes) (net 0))
 (via (at 109.9 100.780152) (size 0.8) (drill 0.4) (layers "F.Cu" "B.Cu") (locked yes) (free yes) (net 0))
 (via (at 124.9 144.180152) (size 0.8) (drill 0.4) (layers "F.Cu" "B.Cu") (locked yes) (free yes) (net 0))
 (via (at 100.7 128.980152) (size 0.8) (drill 0.4) (layers "F.Cu" "B.Cu") (locked yes) (free yes) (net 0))
 (via (at 139.9 100.780152) (size 0.8) (drill 0.4) (layers "F.Cu" "B.Cu") (locked yes) (free yes) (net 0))
 (via (at 144.2 121.480152) (size 0.8) (drill 0.4) (layers "F.Cu" "B.Cu") (locked yes) (free yes) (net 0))
 (via (at 105.4 144.180152) (size 0.8) (drill 0.4) (layers "F.Cu" "B.Cu") (locked yes) (free yes) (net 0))
 (via (at 143.2 142.380152) (size 0.8) (drill 0.4) (layers "F.Cu" "B.Cu") (locked yes) (free yes) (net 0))
 (via (at 136.9 144.180152) (size 0.8) (drill 0.4) (layers "F.Cu" "B.Cu") (locked yes) (free yes) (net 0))
 (via (at 144.2 125.980152) (size 0.8) (drill 0.4) (layers "F.Cu" "B.Cu") (locked yes) (free yes) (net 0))
 (via (at 129.4 100.780152) (size 0.8) (drill 0.4) (layers "F.Cu" "B.Cu") (locked yes) (free yes) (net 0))
 (via (at 100.7 116.980152) (size 0.8) (drill 0.4) (layers "F.Cu" "B.Cu") (locked yes) (free yes) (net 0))
 (segment (start 135.5 117.55) (end 133 120.05) (width 1) (layer "F.Cu") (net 3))
 (segment (start 124.5 116.975) (end 129.925 116.975) (width 1) (layer "F.Cu") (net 3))
 (segment (start 129.925 116.975) (end 133 120.05) (width 1) (layer "F.Cu") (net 3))
 (segment (start 135.5 113.964214) (end 135.5 117.55) (width 1) (layer "F.Cu") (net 3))
 (segment (start 115.5 120.475) (end 114.5 119.475) (width 1) (layer "F.Cu") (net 1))
 (segment (start 106 122) (end 111.975 122) (width 1) (layer "F.Cu") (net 1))
 (segment (start 111.975 122) (end 114.5 119.475) (width 1) (layer "F.Cu") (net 1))
 (segment (start 115.5 130) (end 115.5 120.475) (width 1) (layer "F.Cu") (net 1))
 (segment (start 133 121.95) (end 139.95 121.95) (width 1) (layer "F.Cu") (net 2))
 (segment (start 139.95 121.95) (end 140 122) (width 0.25) (layer "F.Cu") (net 2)))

